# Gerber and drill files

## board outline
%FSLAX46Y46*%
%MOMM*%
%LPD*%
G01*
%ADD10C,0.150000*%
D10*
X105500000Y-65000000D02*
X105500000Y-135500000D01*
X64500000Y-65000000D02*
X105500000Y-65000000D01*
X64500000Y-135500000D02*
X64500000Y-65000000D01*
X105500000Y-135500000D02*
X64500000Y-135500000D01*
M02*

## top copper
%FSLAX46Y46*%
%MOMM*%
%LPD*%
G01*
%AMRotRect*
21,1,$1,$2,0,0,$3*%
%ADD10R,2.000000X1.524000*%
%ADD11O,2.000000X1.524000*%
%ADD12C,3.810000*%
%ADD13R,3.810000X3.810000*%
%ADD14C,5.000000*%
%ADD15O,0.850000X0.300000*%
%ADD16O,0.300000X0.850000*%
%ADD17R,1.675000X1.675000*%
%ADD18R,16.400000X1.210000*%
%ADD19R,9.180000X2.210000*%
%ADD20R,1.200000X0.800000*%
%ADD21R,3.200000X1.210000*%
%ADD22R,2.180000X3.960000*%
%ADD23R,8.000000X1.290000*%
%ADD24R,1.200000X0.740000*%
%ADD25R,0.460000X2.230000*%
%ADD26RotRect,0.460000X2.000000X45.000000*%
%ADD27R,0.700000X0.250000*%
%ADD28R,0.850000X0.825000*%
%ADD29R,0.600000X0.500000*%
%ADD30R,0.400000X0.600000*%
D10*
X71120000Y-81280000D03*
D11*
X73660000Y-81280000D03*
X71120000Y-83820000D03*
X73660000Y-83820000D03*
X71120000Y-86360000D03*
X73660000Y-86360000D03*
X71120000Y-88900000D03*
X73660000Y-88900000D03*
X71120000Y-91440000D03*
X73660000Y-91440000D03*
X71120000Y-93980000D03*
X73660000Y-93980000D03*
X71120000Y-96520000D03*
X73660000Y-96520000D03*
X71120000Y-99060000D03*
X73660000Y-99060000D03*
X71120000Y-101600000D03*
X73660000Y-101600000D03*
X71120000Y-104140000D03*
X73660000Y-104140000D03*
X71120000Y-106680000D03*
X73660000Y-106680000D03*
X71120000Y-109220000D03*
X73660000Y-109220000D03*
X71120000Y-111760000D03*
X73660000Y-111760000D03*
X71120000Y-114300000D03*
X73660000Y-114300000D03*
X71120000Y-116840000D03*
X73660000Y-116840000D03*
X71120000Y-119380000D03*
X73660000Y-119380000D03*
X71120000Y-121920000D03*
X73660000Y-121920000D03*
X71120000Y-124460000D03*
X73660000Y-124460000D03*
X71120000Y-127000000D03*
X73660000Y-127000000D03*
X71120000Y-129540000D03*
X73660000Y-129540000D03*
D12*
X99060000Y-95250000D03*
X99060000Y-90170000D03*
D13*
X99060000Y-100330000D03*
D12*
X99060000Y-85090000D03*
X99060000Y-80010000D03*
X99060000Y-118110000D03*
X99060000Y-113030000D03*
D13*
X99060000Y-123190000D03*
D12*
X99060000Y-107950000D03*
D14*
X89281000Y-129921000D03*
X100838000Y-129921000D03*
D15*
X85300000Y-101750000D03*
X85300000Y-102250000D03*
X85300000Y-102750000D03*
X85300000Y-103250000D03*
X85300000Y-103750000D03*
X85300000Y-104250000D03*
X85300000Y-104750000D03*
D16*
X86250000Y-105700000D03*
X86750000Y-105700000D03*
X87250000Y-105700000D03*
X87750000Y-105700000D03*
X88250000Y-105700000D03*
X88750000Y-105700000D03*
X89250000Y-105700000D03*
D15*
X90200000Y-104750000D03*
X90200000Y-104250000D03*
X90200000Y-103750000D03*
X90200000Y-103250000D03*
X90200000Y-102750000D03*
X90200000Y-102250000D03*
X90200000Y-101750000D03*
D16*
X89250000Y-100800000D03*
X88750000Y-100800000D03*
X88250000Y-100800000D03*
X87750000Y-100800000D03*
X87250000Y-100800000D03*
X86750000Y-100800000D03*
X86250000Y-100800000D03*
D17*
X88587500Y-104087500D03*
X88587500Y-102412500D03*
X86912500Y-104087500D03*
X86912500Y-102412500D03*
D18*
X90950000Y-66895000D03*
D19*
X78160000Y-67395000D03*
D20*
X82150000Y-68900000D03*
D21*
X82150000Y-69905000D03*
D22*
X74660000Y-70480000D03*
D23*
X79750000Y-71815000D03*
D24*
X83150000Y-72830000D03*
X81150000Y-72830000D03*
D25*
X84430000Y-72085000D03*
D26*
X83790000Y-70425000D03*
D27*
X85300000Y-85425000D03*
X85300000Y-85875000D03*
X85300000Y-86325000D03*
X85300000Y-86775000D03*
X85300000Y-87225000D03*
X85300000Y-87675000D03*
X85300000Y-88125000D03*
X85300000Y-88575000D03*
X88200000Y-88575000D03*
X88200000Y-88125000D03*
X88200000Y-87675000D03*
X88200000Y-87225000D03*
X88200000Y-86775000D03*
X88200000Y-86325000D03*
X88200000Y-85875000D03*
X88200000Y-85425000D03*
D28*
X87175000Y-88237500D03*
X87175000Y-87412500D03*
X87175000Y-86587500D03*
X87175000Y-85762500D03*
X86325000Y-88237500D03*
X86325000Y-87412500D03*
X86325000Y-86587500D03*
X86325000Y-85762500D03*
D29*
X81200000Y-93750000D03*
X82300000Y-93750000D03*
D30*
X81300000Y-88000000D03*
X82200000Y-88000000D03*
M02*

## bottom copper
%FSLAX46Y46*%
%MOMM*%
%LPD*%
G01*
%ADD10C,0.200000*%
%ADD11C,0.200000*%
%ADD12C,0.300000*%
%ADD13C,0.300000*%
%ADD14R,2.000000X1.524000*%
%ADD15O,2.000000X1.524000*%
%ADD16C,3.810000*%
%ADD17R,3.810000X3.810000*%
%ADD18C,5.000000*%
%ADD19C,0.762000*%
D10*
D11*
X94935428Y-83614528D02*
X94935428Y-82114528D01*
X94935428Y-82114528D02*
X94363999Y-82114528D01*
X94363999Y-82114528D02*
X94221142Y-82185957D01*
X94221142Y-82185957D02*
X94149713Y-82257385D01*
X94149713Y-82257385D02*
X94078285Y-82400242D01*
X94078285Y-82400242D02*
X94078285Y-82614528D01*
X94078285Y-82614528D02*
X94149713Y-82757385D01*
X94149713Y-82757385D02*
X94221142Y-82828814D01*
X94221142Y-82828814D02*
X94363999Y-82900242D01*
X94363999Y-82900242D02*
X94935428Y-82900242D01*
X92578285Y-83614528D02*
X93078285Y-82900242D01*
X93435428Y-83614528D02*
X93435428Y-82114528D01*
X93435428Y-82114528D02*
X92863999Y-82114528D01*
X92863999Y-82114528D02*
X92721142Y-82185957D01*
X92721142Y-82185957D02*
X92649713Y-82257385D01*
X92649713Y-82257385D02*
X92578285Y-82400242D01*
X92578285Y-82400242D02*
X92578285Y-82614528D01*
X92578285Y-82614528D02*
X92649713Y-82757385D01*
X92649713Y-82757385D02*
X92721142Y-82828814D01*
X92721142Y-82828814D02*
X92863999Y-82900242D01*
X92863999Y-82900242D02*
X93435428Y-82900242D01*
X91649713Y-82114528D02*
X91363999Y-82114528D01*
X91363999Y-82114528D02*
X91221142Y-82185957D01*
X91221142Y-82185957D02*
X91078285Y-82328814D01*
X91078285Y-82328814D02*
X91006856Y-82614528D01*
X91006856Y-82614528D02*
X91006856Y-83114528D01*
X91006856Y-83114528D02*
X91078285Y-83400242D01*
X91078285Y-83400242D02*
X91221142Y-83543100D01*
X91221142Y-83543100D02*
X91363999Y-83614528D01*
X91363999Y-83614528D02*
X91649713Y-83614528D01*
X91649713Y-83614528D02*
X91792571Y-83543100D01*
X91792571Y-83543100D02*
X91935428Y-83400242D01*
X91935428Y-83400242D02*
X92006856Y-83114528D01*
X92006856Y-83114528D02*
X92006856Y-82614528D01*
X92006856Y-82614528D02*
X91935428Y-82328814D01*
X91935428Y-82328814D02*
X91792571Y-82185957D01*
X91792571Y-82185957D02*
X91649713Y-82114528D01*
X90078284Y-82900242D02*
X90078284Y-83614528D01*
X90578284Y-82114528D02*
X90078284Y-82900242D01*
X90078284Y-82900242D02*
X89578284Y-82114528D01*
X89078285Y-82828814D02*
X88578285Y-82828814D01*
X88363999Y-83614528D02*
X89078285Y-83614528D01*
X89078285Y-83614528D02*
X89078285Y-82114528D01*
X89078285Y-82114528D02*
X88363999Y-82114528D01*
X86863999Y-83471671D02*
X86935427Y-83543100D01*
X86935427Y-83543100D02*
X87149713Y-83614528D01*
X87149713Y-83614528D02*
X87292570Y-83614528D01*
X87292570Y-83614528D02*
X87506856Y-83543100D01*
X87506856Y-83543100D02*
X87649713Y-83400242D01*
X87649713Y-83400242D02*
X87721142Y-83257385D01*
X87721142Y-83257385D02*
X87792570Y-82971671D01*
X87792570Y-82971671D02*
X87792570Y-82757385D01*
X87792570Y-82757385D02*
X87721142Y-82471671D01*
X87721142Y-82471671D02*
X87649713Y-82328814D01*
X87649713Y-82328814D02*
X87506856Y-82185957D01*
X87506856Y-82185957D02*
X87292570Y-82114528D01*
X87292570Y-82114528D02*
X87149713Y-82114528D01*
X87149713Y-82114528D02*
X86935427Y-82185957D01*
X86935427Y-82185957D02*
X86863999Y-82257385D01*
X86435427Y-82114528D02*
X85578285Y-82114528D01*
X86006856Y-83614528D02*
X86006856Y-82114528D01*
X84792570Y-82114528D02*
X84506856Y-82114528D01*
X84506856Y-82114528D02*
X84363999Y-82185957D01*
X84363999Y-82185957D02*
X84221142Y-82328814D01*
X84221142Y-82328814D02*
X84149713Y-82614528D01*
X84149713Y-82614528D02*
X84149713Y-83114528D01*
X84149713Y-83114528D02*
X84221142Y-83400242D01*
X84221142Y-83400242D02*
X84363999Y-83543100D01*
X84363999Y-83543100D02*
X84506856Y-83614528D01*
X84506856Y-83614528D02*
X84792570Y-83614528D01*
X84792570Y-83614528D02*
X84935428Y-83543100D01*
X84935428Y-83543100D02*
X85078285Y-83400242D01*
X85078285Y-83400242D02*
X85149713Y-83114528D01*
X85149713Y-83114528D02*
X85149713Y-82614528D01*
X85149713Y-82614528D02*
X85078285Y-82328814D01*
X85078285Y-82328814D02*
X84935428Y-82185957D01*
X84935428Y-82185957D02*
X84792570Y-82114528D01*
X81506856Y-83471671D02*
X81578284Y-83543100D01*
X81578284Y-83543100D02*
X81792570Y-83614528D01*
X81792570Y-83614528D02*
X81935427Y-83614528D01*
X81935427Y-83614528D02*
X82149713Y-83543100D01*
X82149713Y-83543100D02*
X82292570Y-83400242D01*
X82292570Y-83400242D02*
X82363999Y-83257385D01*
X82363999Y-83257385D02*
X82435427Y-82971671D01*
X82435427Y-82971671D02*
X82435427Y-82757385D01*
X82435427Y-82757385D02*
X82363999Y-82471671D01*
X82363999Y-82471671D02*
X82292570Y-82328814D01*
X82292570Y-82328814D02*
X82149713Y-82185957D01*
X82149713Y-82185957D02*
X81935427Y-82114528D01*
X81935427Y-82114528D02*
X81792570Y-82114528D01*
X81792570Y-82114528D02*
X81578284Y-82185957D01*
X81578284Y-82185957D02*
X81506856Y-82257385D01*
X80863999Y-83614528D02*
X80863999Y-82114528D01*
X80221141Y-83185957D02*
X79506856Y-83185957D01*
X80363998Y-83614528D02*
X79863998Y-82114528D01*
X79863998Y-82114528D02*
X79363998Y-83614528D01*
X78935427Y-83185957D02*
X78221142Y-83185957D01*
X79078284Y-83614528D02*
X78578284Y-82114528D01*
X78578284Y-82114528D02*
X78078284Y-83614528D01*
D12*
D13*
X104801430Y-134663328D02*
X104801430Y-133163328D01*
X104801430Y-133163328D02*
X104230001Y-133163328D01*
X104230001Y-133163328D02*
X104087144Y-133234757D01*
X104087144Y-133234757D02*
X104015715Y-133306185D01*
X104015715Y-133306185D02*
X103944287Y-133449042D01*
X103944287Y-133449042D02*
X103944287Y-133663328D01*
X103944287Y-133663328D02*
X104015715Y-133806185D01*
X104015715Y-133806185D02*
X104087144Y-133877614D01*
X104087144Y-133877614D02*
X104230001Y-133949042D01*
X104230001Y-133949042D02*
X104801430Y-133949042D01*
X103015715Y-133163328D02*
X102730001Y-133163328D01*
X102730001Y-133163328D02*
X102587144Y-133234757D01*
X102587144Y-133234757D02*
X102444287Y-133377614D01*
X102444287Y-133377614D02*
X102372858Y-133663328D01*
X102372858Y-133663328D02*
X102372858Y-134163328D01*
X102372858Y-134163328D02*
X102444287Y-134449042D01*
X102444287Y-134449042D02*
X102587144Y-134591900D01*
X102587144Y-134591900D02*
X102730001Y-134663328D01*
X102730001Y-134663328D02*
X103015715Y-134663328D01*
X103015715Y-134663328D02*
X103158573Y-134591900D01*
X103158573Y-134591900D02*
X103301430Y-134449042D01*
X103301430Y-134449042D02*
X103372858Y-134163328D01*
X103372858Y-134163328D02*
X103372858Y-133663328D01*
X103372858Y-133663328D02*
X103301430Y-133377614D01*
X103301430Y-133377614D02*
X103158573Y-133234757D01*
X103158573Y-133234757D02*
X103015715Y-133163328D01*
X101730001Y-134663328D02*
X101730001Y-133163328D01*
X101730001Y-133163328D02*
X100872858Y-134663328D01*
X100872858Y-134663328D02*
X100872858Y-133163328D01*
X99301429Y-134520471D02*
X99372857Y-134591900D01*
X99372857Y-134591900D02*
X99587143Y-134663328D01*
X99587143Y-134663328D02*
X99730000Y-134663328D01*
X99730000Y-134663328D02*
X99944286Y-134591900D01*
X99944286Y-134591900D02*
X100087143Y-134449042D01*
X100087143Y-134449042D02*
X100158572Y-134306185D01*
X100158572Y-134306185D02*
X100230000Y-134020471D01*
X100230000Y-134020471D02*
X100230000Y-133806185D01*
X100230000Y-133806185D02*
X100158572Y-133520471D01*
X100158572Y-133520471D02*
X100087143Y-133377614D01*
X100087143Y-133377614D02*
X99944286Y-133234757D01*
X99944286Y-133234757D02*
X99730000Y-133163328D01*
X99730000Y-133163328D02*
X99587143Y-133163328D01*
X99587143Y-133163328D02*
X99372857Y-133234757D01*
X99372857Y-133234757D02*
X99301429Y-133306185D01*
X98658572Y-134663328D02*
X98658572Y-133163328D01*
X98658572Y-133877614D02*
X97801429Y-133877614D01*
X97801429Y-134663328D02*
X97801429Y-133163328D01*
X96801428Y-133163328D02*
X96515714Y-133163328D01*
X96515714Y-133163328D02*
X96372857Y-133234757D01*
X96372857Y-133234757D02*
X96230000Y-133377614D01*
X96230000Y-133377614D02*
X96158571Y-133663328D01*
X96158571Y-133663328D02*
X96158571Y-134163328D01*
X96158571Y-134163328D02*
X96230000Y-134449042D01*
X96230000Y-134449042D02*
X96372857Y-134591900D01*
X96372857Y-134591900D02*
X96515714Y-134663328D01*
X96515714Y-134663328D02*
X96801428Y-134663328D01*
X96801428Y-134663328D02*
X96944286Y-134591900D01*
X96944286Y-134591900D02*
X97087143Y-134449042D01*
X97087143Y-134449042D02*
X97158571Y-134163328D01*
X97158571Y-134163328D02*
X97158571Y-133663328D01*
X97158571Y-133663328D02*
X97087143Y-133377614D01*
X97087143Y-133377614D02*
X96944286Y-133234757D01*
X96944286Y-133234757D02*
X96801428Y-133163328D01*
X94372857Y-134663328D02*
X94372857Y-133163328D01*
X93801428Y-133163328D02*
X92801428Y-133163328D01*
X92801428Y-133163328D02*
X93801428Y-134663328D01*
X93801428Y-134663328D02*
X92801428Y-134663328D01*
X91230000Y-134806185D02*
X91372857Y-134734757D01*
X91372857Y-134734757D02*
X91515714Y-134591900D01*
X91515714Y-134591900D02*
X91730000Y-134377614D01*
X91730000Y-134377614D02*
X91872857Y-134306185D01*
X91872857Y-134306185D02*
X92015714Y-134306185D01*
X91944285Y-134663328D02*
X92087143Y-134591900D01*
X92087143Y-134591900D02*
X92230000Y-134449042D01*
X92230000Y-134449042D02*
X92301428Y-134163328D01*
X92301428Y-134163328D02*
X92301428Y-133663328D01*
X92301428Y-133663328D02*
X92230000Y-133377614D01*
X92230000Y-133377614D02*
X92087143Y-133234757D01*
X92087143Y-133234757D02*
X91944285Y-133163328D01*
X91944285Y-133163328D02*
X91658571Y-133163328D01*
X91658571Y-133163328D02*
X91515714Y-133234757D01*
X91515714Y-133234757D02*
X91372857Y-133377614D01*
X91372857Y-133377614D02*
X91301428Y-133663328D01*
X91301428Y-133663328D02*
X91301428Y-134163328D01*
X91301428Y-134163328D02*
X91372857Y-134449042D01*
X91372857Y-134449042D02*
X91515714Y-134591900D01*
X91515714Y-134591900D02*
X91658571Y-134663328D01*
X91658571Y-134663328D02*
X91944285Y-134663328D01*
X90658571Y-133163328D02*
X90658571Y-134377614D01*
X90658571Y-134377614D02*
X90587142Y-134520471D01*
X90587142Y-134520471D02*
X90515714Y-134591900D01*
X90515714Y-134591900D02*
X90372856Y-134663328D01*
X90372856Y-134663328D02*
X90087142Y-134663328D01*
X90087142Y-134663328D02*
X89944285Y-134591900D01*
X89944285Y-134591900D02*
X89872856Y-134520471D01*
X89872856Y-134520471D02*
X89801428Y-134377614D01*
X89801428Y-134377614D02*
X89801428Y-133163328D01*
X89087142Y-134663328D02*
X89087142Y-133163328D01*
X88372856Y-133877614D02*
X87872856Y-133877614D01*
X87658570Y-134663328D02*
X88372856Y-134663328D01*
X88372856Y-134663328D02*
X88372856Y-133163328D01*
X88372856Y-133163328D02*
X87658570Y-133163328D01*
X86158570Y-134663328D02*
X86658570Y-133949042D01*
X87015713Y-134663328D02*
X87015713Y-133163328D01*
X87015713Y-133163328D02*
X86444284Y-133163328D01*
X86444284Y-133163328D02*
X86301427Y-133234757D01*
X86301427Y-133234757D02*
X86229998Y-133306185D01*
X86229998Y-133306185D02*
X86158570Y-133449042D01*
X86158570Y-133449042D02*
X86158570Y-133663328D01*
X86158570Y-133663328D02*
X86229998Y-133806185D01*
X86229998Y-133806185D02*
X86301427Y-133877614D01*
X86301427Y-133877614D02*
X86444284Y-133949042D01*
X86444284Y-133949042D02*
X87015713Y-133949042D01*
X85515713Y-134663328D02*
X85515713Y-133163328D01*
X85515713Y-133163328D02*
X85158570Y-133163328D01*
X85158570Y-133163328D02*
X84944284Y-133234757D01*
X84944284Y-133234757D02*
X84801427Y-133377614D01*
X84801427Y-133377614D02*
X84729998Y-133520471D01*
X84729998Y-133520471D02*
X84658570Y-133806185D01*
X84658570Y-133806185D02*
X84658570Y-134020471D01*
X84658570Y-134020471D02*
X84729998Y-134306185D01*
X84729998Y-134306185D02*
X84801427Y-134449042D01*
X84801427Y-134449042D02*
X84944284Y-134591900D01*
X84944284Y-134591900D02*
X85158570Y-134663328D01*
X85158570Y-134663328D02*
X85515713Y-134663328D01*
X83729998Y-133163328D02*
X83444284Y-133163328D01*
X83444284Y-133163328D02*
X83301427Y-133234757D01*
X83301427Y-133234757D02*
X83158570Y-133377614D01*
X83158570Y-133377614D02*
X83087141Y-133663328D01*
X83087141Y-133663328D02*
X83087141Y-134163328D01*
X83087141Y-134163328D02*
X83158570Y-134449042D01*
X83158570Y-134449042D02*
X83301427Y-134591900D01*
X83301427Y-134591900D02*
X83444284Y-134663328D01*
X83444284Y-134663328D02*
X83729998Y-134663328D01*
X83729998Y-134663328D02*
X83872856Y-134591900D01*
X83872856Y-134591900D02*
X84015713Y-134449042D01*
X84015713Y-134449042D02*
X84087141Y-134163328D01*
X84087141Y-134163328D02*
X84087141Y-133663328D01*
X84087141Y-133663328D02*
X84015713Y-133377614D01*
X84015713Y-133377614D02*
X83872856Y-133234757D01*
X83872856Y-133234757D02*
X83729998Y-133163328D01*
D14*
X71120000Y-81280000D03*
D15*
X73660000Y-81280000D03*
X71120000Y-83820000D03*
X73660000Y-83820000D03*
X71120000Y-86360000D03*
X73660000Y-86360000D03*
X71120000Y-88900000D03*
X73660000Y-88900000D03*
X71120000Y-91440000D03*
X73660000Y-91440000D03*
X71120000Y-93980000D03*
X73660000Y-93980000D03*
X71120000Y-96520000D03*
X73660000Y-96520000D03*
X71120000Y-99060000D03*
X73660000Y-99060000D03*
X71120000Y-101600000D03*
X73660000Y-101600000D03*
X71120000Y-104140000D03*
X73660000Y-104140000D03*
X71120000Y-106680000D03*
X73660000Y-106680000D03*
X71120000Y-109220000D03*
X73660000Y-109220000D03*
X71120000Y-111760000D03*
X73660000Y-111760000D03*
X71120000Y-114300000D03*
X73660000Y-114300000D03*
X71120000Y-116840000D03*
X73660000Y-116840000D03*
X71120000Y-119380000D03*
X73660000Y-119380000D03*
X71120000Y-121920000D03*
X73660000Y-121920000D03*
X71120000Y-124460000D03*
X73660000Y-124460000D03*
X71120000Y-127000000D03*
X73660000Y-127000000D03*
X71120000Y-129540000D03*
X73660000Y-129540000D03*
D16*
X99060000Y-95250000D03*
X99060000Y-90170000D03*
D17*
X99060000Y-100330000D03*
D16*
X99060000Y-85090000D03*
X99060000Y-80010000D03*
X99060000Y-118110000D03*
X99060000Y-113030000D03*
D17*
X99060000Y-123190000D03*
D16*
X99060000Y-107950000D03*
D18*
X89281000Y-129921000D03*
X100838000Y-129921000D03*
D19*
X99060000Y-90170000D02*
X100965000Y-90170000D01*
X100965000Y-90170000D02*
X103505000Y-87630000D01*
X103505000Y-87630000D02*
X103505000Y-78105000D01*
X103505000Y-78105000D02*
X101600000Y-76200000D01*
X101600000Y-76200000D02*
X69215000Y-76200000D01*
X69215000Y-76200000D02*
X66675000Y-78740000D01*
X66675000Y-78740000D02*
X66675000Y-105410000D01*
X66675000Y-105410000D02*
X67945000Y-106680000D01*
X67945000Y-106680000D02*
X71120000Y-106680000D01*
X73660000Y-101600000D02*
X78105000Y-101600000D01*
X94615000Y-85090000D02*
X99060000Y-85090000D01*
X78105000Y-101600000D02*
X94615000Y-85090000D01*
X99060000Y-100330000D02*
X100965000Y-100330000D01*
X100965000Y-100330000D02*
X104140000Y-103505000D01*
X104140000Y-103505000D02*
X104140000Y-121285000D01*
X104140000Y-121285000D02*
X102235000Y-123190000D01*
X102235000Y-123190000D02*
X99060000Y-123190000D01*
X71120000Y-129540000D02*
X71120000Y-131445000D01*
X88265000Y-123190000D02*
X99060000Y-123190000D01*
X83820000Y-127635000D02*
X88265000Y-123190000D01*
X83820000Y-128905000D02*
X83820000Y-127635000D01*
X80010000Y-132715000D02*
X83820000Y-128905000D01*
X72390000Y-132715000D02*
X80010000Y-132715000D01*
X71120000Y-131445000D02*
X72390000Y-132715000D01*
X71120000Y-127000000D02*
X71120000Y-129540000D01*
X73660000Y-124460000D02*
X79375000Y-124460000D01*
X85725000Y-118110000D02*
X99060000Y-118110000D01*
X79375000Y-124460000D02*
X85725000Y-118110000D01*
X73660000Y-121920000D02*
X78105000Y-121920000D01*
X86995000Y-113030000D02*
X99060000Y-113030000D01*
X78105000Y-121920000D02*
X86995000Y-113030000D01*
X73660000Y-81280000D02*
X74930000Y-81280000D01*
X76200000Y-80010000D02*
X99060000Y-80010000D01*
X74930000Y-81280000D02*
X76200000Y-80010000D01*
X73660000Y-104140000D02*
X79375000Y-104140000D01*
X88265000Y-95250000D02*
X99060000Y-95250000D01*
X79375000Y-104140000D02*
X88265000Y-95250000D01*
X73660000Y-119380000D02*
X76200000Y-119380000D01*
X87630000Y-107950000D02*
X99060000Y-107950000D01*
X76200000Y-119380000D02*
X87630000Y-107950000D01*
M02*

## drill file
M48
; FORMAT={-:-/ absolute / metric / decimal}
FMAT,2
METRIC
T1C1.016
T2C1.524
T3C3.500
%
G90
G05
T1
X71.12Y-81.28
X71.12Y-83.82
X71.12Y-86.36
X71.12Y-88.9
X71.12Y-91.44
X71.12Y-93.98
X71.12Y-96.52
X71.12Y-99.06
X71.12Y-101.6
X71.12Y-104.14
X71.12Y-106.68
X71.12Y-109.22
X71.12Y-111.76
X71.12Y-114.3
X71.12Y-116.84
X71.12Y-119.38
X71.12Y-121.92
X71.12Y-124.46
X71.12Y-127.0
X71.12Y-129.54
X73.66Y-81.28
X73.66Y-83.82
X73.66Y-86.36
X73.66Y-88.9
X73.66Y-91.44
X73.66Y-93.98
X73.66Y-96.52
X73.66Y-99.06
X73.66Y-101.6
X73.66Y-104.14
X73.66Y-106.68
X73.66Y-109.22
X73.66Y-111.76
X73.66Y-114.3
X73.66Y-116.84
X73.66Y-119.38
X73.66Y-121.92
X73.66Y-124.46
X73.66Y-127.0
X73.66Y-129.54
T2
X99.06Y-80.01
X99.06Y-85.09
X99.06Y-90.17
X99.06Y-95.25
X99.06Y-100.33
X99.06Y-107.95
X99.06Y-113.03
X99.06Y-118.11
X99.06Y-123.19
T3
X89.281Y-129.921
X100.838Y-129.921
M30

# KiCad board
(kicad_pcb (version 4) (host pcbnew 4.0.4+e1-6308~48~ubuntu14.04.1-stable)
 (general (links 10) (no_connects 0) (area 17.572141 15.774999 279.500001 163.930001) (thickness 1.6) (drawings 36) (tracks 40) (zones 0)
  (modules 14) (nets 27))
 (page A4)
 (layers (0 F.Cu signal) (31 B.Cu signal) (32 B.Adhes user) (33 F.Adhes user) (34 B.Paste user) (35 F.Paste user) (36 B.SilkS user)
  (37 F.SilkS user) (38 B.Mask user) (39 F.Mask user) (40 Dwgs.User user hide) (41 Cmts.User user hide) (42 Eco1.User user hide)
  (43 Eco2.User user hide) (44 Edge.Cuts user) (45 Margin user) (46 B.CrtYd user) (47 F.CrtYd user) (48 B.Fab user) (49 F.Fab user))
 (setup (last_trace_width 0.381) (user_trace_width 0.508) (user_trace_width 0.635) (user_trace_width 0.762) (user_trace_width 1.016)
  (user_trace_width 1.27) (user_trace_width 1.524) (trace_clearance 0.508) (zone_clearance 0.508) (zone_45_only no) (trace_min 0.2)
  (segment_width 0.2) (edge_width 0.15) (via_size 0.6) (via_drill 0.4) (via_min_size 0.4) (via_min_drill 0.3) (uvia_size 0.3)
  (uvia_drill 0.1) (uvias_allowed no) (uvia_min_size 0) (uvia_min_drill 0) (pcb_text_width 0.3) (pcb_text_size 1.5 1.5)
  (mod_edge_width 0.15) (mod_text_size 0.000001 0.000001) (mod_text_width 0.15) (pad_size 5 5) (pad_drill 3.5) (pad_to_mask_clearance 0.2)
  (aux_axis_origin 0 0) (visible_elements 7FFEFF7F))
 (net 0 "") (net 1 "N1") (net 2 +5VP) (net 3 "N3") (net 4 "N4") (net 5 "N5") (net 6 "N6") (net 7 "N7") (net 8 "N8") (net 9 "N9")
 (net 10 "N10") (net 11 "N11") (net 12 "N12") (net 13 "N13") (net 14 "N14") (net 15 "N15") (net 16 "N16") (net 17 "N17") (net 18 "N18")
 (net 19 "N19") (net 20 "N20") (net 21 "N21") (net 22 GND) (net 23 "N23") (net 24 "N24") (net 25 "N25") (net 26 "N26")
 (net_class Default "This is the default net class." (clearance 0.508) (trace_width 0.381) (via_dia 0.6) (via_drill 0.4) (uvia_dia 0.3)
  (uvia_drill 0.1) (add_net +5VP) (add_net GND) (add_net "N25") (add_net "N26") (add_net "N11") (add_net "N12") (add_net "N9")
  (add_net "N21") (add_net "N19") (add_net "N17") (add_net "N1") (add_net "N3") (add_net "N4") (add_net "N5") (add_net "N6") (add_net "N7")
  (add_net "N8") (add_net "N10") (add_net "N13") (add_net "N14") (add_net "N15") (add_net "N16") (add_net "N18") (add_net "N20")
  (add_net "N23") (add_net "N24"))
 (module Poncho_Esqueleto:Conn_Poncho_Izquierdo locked (layer F.Cu) (at 71.12 81.28)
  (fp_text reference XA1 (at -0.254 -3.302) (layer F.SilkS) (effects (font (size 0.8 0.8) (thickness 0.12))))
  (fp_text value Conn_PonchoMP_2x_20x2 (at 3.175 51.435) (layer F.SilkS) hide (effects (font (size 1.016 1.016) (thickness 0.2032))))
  (pad 41 thru_hole rect (at 0 0 270) (size 1.524 2) (drill 1.016) (layers *.Cu *.Mask F.SilkS) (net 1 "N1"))
  (pad 42 thru_hole oval (at 2.54 0 270) (size 1.524 2) (drill 1.016) (layers *.Cu *.Mask F.SilkS) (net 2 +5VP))
  (pad 43 thru_hole oval (at 0 2.54 270) (size 1.524 2) (drill 1.016) (layers *.Cu *.Mask F.SilkS) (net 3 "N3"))
  (pad 44 thru_hole oval (at 2.54 2.54 270) (size 1.524 2) (drill 1.016) (layers *.Cu *.Mask F.SilkS))
  (pad 45 thru_hole oval (at 0 5.08 270) (size 1.524 2) (drill 1.016) (layers *.Cu *.Mask F.SilkS) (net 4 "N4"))
  (pad 46 thru_hole oval (at 2.54 5.08 270) (size 1.524 2) (drill 1.016) (layers *.Cu *.Mask F.SilkS))
  (pad 47 thru_hole oval (at 0 7.62 270) (size 1.524 2) (drill 1.016) (layers *.Cu *.Mask F.SilkS) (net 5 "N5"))
  (pad 48 thru_hole oval (at 2.54 7.62 270) (size 1.524 2) (drill 1.016) (layers *.Cu *.Mask F.SilkS))
  (pad 49 thru_hole oval (at 0 10.16 270) (size 1.524 2) (drill 1.016) (layers *.Cu *.Mask F.SilkS))
  (pad 50 thru_hole oval (at 2.54 10.16 270) (size 1.524 2) (drill 1.016) (layers *.Cu *.Mask F.SilkS))
  (pad 51 thru_hole oval (at 0 12.7 270) (size 1.524 2) (drill 1.016) (layers *.Cu *.Mask F.SilkS) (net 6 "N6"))
  (pad 52 thru_hole oval (at 2.54 12.7 270) (size 1.524 2) (drill 1.016) (layers *.Cu *.Mask F.SilkS))
  (pad 53 thru_hole oval (at 0 15.24 270) (size 1.524 2) (drill 1.016) (layers *.Cu *.Mask F.SilkS) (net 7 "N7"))
  (pad 54 thru_hole oval (at 2.54 15.24 270) (size 1.524 2) (drill 1.016) (layers *.Cu *.Mask F.SilkS))
  (pad 55 thru_hole oval (at 0 17.78 270) (size 1.524 2) (drill 1.016) (layers *.Cu *.Mask F.SilkS))
  (pad 56 thru_hole oval (at 2.54 17.78 270) (size 1.524 2) (drill 1.016) (layers *.Cu *.Mask F.SilkS))
  (pad 57 thru_hole oval (at 0 20.32 270) (size 1.524 2) (drill 1.016) (layers *.Cu *.Mask F.SilkS) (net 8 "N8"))
  (pad 58 thru_hole oval (at 2.54 20.32 270) (size 1.524 2) (drill 1.016) (layers *.Cu *.Mask F.SilkS) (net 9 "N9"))
  (pad 59 thru_hole oval (at 0 22.86 270) (size 1.524 2) (drill 1.016) (layers *.Cu *.Mask F.SilkS) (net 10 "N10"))
  (pad 60 thru_hole oval (at 2.54 22.86 270) (size 1.524 2) (drill 1.016) (layers *.Cu *.Mask F.SilkS) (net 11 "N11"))
  (pad 61 thru_hole oval (at 0 25.4 270) (size 1.524 2) (drill 1.016) (layers *.Cu *.Mask F.SilkS) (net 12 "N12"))
  (pad 62 thru_hole oval (at 2.54 25.4 270) (size 1.524 2) (drill 1.016) (layers *.Cu *.Mask F.SilkS))
  (pad 63 thru_hole oval (at 0 27.94 270) (size 1.524 2) (drill 1.016) (layers *.Cu *.Mask F.SilkS))
  (pad 64 thru_hole oval (at 2.54 27.94 270) (size 1.524 2) (drill 1.016) (layers *.Cu *.Mask F.SilkS))
  (pad 65 thru_hole oval (at 0 30.48 270) (size 1.524 2) (drill 1.016) (layers *.Cu *.Mask F.SilkS) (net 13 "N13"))
  (pad 66 thru_hole oval (at 2.54 30.48 270) (size 1.524 2) (drill 1.016) (layers *.Cu *.Mask F.SilkS))
  (pad 67 thru_hole oval (at 0 33.02 270) (size 1.524 2) (drill 1.016) (layers *.Cu *.Mask F.SilkS) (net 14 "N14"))
  (pad 68 thru_hole oval (at 2.54 33.02 270) (size 1.524 2) (drill 1.016) (layers *.Cu *.Mask F.SilkS))
  (pad 69 thru_hole oval (at 0 35.56 270) (size 1.524 2) (drill 1.016) (layers *.Cu *.Mask F.SilkS) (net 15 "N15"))
  (pad 70 thru_hole oval (at 2.54 35.56 270) (size 1.524 2) (drill 1.016) (layers *.Cu *.Mask F.SilkS))
  (pad 71 thru_hole oval (at 0 38.1 270) (size 1.524 2) (drill 1.016) (layers *.Cu *.Mask F.SilkS) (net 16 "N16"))
  (pad 72 thru_hole oval (at 2.54 38.1 270) (size 1.524 2) (drill 1.016) (layers *.Cu *.Mask F.SilkS) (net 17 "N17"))
  (pad 73 thru_hole oval (at 0 40.64 270) (size 1.524 2) (drill 1.016) (layers *.Cu *.Mask F.SilkS) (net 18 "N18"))
  (pad 74 thru_hole oval (at 2.54 40.64 270) (size 1.524 2) (drill 1.016) (layers *.Cu *.Mask F.SilkS) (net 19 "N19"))
  (pad 75 thru_hole oval (at 0 43.18 270) (size 1.524 2) (drill 1.016) (layers *.Cu *.Mask F.SilkS) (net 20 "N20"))
  (pad 76 thru_hole oval (at 2.54 43.18 270) (size 1.524 2) (drill 1.016) (layers *.Cu *.Mask F.SilkS) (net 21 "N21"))
  (pad 77 thru_hole oval (at 0 45.72 270) (size 1.524 2) (drill 1.016) (layers *.Cu *.Mask F.SilkS) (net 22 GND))
  (pad 78 thru_hole oval (at 2.54 45.72 270) (size 1.524 2) (drill 1.016) (layers *.Cu *.Mask F.SilkS) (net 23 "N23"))
  (pad 79 thru_hole oval (at 0 48.26 270) (size 1.524 2) (drill 1.016) (layers *.Cu *.Mask F.SilkS) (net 22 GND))
  (pad 80 thru_hole oval (at 2.54 48.26 270) (size 1.524 2) (drill 1.016) (layers *.Cu *.Mask F.SilkS) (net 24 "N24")))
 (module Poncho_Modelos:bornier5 (layer F.Cu) (at 99.06 90.17 90)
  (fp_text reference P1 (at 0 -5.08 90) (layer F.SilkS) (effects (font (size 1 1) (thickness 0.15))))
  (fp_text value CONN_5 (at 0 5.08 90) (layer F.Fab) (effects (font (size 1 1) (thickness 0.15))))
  (pad 2 thru_hole circle (at -5.08 0 90) (size 3.81 3.81) (drill 1.524) (layers *.Cu *.Mask F.SilkS) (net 11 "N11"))
  (pad 3 thru_hole circle (at 0 0 90) (size 3.81 3.81) (drill 1.524) (layers *.Cu *.Mask F.SilkS) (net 12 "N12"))
  (pad 1 thru_hole rect (at -10.16 0 90) (size 3.81 3.81) (drill 1.524) (layers *.Cu *.Mask F.SilkS) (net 22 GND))
  (pad 4 thru_hole circle (at 5.08 0 90) (size 3.81 3.81) (drill 1.524) (layers *.Cu *.Mask F.SilkS) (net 9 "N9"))
  (pad 5 thru_hole circle (at 10.16 0 90) (size 3.81 3.81) (drill 1.524) (layers *.Cu *.Mask F.SilkS) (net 2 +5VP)))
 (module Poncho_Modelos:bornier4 (layer F.Cu) (at 99.06 115.57 90)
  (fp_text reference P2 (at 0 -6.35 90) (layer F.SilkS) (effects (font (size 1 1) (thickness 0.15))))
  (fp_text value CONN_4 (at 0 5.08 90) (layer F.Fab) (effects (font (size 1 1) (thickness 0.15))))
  (pad 2 thru_hole circle (at -2.54 0 90) (size 3.81 3.81) (drill 1.524) (layers *.Cu *.Mask F.SilkS) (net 21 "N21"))
  (pad 3 thru_hole circle (at 2.54 0 90) (size 3.81 3.81) (drill 1.524) (layers *.Cu *.Mask F.SilkS) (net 19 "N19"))
  (pad 1 thru_hole rect (at -7.62 0 90) (size 3.81 3.81) (drill 1.524) (layers *.Cu *.Mask F.SilkS) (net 22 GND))
  (pad 4 thru_hole circle (at 7.62 0 90) (size 3.81 3.81) (drill 1.524) (layers *.Cu *.Mask F.SilkS) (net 17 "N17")))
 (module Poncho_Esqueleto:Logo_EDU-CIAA (layer F.Cu) (at 87.5 112.25)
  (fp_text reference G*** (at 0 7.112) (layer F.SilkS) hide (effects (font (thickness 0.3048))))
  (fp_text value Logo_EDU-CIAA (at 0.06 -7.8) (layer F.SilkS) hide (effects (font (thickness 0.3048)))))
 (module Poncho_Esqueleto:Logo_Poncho (layer F.Cu) (at 87.25 94.25)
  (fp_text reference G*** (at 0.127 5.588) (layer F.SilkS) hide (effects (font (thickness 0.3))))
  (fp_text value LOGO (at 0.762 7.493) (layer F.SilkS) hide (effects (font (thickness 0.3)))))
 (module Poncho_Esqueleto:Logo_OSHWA (layer F.Cu) (at 87 123)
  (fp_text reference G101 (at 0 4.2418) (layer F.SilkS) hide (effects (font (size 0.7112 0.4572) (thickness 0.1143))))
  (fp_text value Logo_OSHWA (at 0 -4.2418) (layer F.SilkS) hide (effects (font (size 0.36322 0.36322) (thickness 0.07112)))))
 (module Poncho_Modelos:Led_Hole (layer F.Cu) (at 89.281 129.921)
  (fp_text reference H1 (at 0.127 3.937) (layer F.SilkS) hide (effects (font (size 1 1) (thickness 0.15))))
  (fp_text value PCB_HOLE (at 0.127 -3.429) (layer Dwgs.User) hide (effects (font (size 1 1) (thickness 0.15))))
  (pad 1 thru_hole circle (at 0 0) (size 5 5) (drill 3.5) (layers *.Cu *.Mask F.SilkS) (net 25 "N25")))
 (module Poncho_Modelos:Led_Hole (layer F.Cu) (at 100.838 129.921)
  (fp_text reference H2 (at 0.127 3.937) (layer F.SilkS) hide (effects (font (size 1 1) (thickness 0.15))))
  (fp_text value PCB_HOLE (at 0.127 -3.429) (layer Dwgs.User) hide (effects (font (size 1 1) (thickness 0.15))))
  (pad 1 thru_hole circle (at 0 0) (size 5 5) (drill 3.5) (layers *.Cu *.Mask F.SilkS) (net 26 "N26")))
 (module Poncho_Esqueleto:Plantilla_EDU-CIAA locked (layer F.Cu) (at 142.24 81.28)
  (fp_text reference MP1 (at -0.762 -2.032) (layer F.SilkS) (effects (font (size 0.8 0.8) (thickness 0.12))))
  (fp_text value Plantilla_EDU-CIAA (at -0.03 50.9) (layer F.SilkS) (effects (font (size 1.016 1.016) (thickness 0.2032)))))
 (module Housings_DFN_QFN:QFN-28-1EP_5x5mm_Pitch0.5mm (layer F.Cu) (at 87.75 103.25)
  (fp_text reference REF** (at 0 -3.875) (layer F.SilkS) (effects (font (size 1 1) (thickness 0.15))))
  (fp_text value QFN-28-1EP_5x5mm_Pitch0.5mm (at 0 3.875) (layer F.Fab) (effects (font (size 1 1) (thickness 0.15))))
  (pad 1 smd oval (at -2.45 -1.5) (size 0.85 0.3) (layers F.Cu F.Paste F.Mask))
  (pad 2 smd oval (at -2.45 -1) (size 0.85 0.3) (layers F.Cu F.Paste F.Mask))
  (pad 3 smd oval (at -2.45 -0.5) (size 0.85 0.3) (layers F.Cu F.Paste F.Mask))
  (pad 4 smd oval (at -2.45 0) (size 0.85 0.3) (layers F.Cu F.Paste F.Mask))
  (pad 5 smd oval (at -2.45 0.5) (size 0.85 0.3) (layers F.Cu F.Paste F.Mask))
  (pad 6 smd oval (at -2.45 1) (size 0.85 0.3) (layers F.Cu F.Paste F.Mask))
  (pad 7 smd oval (at -2.45 1.5) (size 0.85 0.3) (layers F.Cu F.Paste F.Mask))
  (pad 8 smd oval (at -1.5 2.45 90) (size 0.85 0.3) (layers F.Cu F.Paste F.Mask))
  (pad 9 smd oval (at -1 2.45 90) (size 0.85 0.3) (layers F.Cu F.Paste F.Mask))
  (pad 10 smd oval (at -0.5 2.45 90) (size 0.85 0.3) (layers F.Cu F.Paste F.Mask))
  (pad 11 smd oval (at 0 2.45 90) (size 0.85 0.3) (layers F.Cu F.Paste F.Mask))
  (pad 12 smd oval (at 0.5 2.45 90) (size 0.85 0.3) (layers F.Cu F.Paste F.Mask))
  (pad 13 smd oval (at 1 2.45 90) (size 0.85 0.3) (layers F.Cu F.Paste F.Mask))
  (pad 14 smd oval (at 1.5 2.45 90) (size 0.85 0.3) (layers F.Cu F.Paste F.Mask))
  (pad 15 smd oval (at 2.45 1.5) (size 0.85 0.3) (layers F.Cu F.Paste F.Mask))
  (pad 16 smd oval (at 2.45 1) (size 0.85 0.3) (layers F.Cu F.Paste F.Mask))
  (pad 17 smd oval (at 2.45 0.5) (size 0.85 0.3) (layers F.Cu F.Paste F.Mask))
  (pad 18 smd oval (at 2.45 0) (size 0.85 0.3) (layers F.Cu F.Paste F.Mask))
  (pad 19 smd oval (at 2.45 -0.5) (size 0.85 0.3) (layers F.Cu F.Paste F.Mask))
  (pad 20 smd oval (at 2.45 -1) (size 0.85 0.3) (layers F.Cu F.Paste F.Mask))
  (pad 21 smd oval (at 2.45 -1.5) (size 0.85 0.3) (layers F.Cu F.Paste F.Mask))
  (pad 22 smd oval (at 1.5 -2.45 90) (size 0.85 0.3) (layers F.Cu F.Paste F.Mask))
  (pad 23 smd oval (at 1 -2.45 90) (size 0.85 0.3) (layers F.Cu F.Paste F.Mask))
  (pad 24 smd oval (at 0.5 -2.45 90) (size 0.85 0.3) (layers F.Cu F.Paste F.Mask))
  (pad 25 smd oval (at 0 -2.45 90) (size 0.85 0.3) (layers F.Cu F.Paste F.Mask))
  (pad 26 smd oval (at -0.5 -2.45 90) (size 0.85 0.3) (layers F.Cu F.Paste F.Mask))
  (pad 27 smd oval (at -1 -2.45 90) (size 0.85 0.3) (layers F.Cu F.Paste F.Mask))
  (pad 28 smd oval (at -1.5 -2.45 90) (size 0.85 0.3) (layers F.Cu F.Paste F.Mask))
  (pad 29 smd rect (at 0.8375 0.8375) (size 1.675 1.675) (layers F.Cu F.Paste F.Mask) (solder_paste_margin_ratio -0.2))
  (pad 29 smd rect (at 0.8375 -0.8375) (size 1.675 1.675) (layers F.Cu F.Paste F.Mask) (solder_paste_margin_ratio -0.2))
  (pad 29 smd rect (at -0.8375 0.8375) (size 1.675 1.675) (layers F.Cu F.Paste F.Mask) (solder_paste_margin_ratio -0.2))
  (pad 29 smd rect (at -0.8375 -0.8375) (size 1.675 1.675) (layers F.Cu F.Paste F.Mask) (solder_paste_margin_ratio -0.2)))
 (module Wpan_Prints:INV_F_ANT (layer F.Cu) (at 82.75 67.5)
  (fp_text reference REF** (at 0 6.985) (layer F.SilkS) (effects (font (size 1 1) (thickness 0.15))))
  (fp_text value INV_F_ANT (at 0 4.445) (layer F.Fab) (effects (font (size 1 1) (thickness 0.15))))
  (pad "" smd rect (at 8.2 -0.605) (size 16.4 1.21) (layers F.Cu F.Paste))
  (pad "" smd rect (at -4.59 -0.105) (size 9.18 2.21) (layers F.Cu F.Paste))
  (pad "" smd rect (at -0.6 1.4) (size 1.2 0.8) (layers F.Cu F.Paste))
  (pad "" smd rect (at -0.6 2.405) (size 3.2 1.21) (layers F.Cu F.Paste))
  (pad "" smd rect (at -8.09 2.98) (size 2.18 3.96) (layers F.Cu F.Paste))
  (pad "" smd rect (at -3 4.315) (size 8 1.29) (layers F.Cu F.Paste))
  (pad 2 smd rect (at 0.4 5.33) (size 1.2 0.74) (layers F.Cu F.Paste) (zone_connect 2))
  (pad 3 smd rect (at -1.6 5.33) (size 1.2 0.74) (layers F.Cu F.Paste) (zone_connect 2))
  (pad 1 smd rect (at 1.68 4.585) (size 0.46 2.23) (layers F.Cu F.Paste))
  (pad "" smd rect (at 1.04 2.925 45) (size 0.46 2) (layers F.Cu F.Paste)))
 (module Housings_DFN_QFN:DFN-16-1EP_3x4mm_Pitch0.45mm (layer F.Cu) (at 86.75 87)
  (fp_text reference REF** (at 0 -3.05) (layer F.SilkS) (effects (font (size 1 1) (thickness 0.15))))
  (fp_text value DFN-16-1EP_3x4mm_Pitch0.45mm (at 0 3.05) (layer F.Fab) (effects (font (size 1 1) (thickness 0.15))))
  (pad 1 smd rect (at -1.45 -1.575) (size 0.7 0.25) (layers F.Cu F.Paste F.Mask))
  (pad 2 smd rect (at -1.45 -1.125) (size 0.7 0.25) (layers F.Cu F.Paste F.Mask))
  (pad 3 smd rect (at -1.45 -0.675) (size 0.7 0.25) (layers F.Cu F.Paste F.Mask))
  (pad 4 smd rect (at -1.45 -0.225) (size 0.7 0.25) (layers F.Cu F.Paste F.Mask))
  (pad 5 smd rect (at -1.45 0.225) (size 0.7 0.25) (layers F.Cu F.Paste F.Mask))
  (pad 6 smd rect (at -1.45 0.675) (size 0.7 0.25) (layers F.Cu F.Paste F.Mask))
  (pad 7 smd rect (at -1.45 1.125) (size 0.7 0.25) (layers F.Cu F.Paste F.Mask))
  (pad 8 smd rect (at -1.45 1.575) (size 0.7 0.25) (layers F.Cu F.Paste F.Mask))
  (pad 9 smd rect (at 1.45 1.575) (size 0.7 0.25) (layers F.Cu F.Paste F.Mask))
  (pad 10 smd rect (at 1.45 1.125) (size 0.7 0.25) (layers F.Cu F.Paste F.Mask))
  (pad 11 smd rect (at 1.45 0.675) (size 0.7 0.25) (layers F.Cu F.Paste F.Mask))
  (pad 12 smd rect (at 1.45 0.225) (size 0.7 0.25) (layers F.Cu F.Paste F.Mask))
  (pad 13 smd rect (at 1.45 -0.225) (size 0.7 0.25) (layers F.Cu F.Paste F.Mask))
  (pad 14 smd rect (at 1.45 -0.675) (size 0.7 0.25) (layers F.Cu F.Paste F.Mask))
  (pad 15 smd rect (at 1.45 -1.125) (size 0.7 0.25) (layers F.Cu F.Paste F.Mask))
  (pad 16 smd rect (at 1.45 -1.575) (size 0.7 0.25) (layers F.Cu F.Paste F.Mask))
  (pad 17 smd rect (at 0.425 1.2375) (size 0.85 0.825) (layers F.Cu F.Paste F.Mask) (solder_paste_margin_ratio -0.2))
  (pad 17 smd rect (at 0.425 0.4125) (size 0.85 0.825) (layers F.Cu F.Paste F.Mask) (solder_paste_margin_ratio -0.2))
  (pad 17 smd rect (at 0.425 -0.4125) (size 0.85 0.825) (layers F.Cu F.Paste F.Mask) (solder_paste_margin_ratio -0.2))
  (pad 17 smd rect (at 0.425 -1.2375) (size 0.85 0.825) (layers F.Cu F.Paste F.Mask) (solder_paste_margin_ratio -0.2))
  (pad 17 smd rect (at -0.425 1.2375) (size 0.85 0.825) (layers F.Cu F.Paste F.Mask) (solder_paste_margin_ratio -0.2))
  (pad 17 smd rect (at -0.425 0.4125) (size 0.85 0.825) (layers F.Cu F.Paste F.Mask) (solder_paste_margin_ratio -0.2))
  (pad 17 smd rect (at -0.425 -0.4125) (size 0.85 0.825) (layers F.Cu F.Paste F.Mask) (solder_paste_margin_ratio -0.2))
  (pad 17 smd rect (at -0.425 -1.2375) (size 0.85 0.825) (layers F.Cu F.Paste F.Mask) (solder_paste_margin_ratio -0.2)))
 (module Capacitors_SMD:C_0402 (layer F.Cu) (at 81.75 93.75)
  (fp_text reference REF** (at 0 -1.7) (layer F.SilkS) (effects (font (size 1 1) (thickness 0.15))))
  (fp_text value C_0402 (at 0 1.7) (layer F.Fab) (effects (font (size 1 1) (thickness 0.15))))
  (pad 1 smd rect (at -0.55 0) (size 0.6 0.5) (layers F.Cu F.Paste F.Mask))
  (pad 2 smd rect (at 0.55 0) (size 0.6 0.5) (layers F.Cu F.Paste F.Mask)))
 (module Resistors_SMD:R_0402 (layer F.Cu) (at 81.75 88)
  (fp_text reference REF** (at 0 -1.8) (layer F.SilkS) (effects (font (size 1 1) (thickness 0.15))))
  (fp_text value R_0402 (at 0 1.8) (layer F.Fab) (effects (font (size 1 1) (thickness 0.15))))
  (pad 1 smd rect (at -0.45 0) (size 0.4 0.6) (layers F.Cu F.Paste F.Mask))
  (pad 2 smd rect (at 0.45 0) (size 0.4 0.6) (layers F.Cu F.Paste F.Mask)))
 (gr_line (start 105.5 65) (end 105.5 135.5) (angle 90) (layer Edge.Cuts) (width 0.15))
 (gr_line (start 64.5 65) (end 105.5 65) (angle 90) (layer Edge.Cuts) (width 0.15))
 (gr_line (start 64.5 135.5) (end 64.5 65) (angle 90) (layer Edge.Cuts) (width 0.15))
 (gr_line (start 105.5 135.5) (end 64.5 135.5) (angle 90) (layer Edge.Cuts) (width 0.15))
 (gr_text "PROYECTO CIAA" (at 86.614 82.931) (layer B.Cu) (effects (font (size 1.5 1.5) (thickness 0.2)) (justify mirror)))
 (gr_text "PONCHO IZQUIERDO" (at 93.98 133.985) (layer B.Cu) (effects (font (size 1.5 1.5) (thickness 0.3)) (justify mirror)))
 (segment (start 99.06 90.17) (end 100.965 90.17) (width 0.762) (layer B.Cu) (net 12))
 (segment (start 100.965 90.17) (end 103.505 87.63) (width 0.762) (layer B.Cu) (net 12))
 (segment (start 103.505 87.63) (end 103.505 78.105) (width 0.762) (layer B.Cu) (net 12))
 (segment (start 103.505 78.105) (end 101.6 76.2) (width 0.762) (layer B.Cu) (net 12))
 (segment (start 101.6 76.2) (end 69.215 76.2) (width 0.762) (layer B.Cu) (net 12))
 (segment (start 69.215 76.2) (end 66.675 78.74) (width 0.762) (layer B.Cu) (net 12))
 (segment (start 66.675 78.74) (end 66.675 105.41) (width 0.762) (layer B.Cu) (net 12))
 (segment (start 66.675 105.41) (end 67.945 106.68) (width 0.762) (layer B.Cu) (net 12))
 (segment (start 67.945 106.68) (end 71.12 106.68) (width 0.762) (layer B.Cu) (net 12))
 (segment (start 73.66 101.6) (end 78.105 101.6) (width 0.762) (layer B.Cu) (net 9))
 (segment (start 94.615 85.09) (end 99.06 85.09) (width 0.762) (layer B.Cu) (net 9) (status 20))
 (segment (start 78.105 101.6) (end 94.615 85.09) (width 0.762) (layer B.Cu) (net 9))
 (segment (start 99.06 100.33) (end 100.965 100.33) (width 0.762) (layer B.Cu) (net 22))
 (segment (start 100.965 100.33) (end 104.14 103.505) (width 0.762) (layer B.Cu) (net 22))
 (segment (start 104.14 103.505) (end 104.14 121.285) (width 0.762) (layer B.Cu) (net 22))
 (segment (start 104.14 121.285) (end 102.235 123.19) (width 0.762) (layer B.Cu) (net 22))
 (segment (start 102.235 123.19) (end 99.06 123.19) (width 0.762) (layer B.Cu) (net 22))
 (segment (start 71.12 129.54) (end 71.12 131.445) (width 0.762) (layer B.Cu) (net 22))
 (segment (start 88.265 123.19) (end 99.06 123.19) (width 0.762) (layer B.Cu) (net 22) (status 20))
 (segment (start 83.82 127.635) (end 88.265 123.19) (width 0.762) (layer B.Cu) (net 22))
 (segment (start 83.82 128.905) (end 83.82 127.635) (width 0.762) (layer B.Cu) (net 22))
 (segment (start 80.01 132.715) (end 83.82 128.905) (width 0.762) (layer B.Cu) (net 22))
 (segment (start 72.39 132.715) (end 80.01 132.715) (width 0.762) (layer B.Cu) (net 22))
 (segment (start 71.12 131.445) (end 72.39 132.715) (width 0.762) (layer B.Cu) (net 22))
 (segment (start 71.12 127) (end 71.12 129.54) (width 0.762) (layer B.Cu) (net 22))
 (segment (start 73.66 124.46) (end 79.375 124.46) (width 0.762) (layer B.Cu) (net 21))
 (segment (start 85.725 118.11) (end 99.06 118.11) (width 0.762) (layer B.Cu) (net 21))
 (segment (start 79.375 124.46) (end 85.725 118.11) (width 0.762) (layer B.Cu) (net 21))
 (segment (start 73.66 121.92) (end 78.105 121.92) (width 0.762) (layer B.Cu) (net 19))
 (segment (start 86.995 113.03) (end 99.06 113.03) (width 0.762) (layer B.Cu) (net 19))
 (segment (start 78.105 121.92) (end 86.995 113.03) (width 0.762) (layer B.Cu) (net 19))
 (segment (start 73.66 81.28) (end 74.93 81.28) (width 0.762) (layer B.Cu) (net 2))
 (segment (start 76.2 80.01) (end 99.06 80.01) (width 0.762) (layer B.Cu) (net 2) (status 20))
 (segment (start 74.93 81.28) (end 76.2 80.01) (width 0.762) (layer B.Cu) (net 2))
 (segment (start 73.66 104.14) (end 79.375 104.14) (width 0.762) (layer B.Cu) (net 11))
 (segment (start 88.265 95.25) (end 99.06 95.25) (width 0.762) (layer B.Cu) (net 11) (status 20))
 (segment (start 79.375 104.14) (end 88.265 95.25) (width 0.762) (layer B.Cu) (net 11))
 (segment (start 73.66 119.38) (end 76.2 119.38) (width 0.762) (layer B.Cu) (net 17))
 (segment (start 87.63 107.95) (end 99.06 107.95) (width 0.762) (layer B.Cu) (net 17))
 (segment (start 76.2 119.38) (end 87.63 107.95) (width 0.762) (layer B.Cu) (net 17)))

